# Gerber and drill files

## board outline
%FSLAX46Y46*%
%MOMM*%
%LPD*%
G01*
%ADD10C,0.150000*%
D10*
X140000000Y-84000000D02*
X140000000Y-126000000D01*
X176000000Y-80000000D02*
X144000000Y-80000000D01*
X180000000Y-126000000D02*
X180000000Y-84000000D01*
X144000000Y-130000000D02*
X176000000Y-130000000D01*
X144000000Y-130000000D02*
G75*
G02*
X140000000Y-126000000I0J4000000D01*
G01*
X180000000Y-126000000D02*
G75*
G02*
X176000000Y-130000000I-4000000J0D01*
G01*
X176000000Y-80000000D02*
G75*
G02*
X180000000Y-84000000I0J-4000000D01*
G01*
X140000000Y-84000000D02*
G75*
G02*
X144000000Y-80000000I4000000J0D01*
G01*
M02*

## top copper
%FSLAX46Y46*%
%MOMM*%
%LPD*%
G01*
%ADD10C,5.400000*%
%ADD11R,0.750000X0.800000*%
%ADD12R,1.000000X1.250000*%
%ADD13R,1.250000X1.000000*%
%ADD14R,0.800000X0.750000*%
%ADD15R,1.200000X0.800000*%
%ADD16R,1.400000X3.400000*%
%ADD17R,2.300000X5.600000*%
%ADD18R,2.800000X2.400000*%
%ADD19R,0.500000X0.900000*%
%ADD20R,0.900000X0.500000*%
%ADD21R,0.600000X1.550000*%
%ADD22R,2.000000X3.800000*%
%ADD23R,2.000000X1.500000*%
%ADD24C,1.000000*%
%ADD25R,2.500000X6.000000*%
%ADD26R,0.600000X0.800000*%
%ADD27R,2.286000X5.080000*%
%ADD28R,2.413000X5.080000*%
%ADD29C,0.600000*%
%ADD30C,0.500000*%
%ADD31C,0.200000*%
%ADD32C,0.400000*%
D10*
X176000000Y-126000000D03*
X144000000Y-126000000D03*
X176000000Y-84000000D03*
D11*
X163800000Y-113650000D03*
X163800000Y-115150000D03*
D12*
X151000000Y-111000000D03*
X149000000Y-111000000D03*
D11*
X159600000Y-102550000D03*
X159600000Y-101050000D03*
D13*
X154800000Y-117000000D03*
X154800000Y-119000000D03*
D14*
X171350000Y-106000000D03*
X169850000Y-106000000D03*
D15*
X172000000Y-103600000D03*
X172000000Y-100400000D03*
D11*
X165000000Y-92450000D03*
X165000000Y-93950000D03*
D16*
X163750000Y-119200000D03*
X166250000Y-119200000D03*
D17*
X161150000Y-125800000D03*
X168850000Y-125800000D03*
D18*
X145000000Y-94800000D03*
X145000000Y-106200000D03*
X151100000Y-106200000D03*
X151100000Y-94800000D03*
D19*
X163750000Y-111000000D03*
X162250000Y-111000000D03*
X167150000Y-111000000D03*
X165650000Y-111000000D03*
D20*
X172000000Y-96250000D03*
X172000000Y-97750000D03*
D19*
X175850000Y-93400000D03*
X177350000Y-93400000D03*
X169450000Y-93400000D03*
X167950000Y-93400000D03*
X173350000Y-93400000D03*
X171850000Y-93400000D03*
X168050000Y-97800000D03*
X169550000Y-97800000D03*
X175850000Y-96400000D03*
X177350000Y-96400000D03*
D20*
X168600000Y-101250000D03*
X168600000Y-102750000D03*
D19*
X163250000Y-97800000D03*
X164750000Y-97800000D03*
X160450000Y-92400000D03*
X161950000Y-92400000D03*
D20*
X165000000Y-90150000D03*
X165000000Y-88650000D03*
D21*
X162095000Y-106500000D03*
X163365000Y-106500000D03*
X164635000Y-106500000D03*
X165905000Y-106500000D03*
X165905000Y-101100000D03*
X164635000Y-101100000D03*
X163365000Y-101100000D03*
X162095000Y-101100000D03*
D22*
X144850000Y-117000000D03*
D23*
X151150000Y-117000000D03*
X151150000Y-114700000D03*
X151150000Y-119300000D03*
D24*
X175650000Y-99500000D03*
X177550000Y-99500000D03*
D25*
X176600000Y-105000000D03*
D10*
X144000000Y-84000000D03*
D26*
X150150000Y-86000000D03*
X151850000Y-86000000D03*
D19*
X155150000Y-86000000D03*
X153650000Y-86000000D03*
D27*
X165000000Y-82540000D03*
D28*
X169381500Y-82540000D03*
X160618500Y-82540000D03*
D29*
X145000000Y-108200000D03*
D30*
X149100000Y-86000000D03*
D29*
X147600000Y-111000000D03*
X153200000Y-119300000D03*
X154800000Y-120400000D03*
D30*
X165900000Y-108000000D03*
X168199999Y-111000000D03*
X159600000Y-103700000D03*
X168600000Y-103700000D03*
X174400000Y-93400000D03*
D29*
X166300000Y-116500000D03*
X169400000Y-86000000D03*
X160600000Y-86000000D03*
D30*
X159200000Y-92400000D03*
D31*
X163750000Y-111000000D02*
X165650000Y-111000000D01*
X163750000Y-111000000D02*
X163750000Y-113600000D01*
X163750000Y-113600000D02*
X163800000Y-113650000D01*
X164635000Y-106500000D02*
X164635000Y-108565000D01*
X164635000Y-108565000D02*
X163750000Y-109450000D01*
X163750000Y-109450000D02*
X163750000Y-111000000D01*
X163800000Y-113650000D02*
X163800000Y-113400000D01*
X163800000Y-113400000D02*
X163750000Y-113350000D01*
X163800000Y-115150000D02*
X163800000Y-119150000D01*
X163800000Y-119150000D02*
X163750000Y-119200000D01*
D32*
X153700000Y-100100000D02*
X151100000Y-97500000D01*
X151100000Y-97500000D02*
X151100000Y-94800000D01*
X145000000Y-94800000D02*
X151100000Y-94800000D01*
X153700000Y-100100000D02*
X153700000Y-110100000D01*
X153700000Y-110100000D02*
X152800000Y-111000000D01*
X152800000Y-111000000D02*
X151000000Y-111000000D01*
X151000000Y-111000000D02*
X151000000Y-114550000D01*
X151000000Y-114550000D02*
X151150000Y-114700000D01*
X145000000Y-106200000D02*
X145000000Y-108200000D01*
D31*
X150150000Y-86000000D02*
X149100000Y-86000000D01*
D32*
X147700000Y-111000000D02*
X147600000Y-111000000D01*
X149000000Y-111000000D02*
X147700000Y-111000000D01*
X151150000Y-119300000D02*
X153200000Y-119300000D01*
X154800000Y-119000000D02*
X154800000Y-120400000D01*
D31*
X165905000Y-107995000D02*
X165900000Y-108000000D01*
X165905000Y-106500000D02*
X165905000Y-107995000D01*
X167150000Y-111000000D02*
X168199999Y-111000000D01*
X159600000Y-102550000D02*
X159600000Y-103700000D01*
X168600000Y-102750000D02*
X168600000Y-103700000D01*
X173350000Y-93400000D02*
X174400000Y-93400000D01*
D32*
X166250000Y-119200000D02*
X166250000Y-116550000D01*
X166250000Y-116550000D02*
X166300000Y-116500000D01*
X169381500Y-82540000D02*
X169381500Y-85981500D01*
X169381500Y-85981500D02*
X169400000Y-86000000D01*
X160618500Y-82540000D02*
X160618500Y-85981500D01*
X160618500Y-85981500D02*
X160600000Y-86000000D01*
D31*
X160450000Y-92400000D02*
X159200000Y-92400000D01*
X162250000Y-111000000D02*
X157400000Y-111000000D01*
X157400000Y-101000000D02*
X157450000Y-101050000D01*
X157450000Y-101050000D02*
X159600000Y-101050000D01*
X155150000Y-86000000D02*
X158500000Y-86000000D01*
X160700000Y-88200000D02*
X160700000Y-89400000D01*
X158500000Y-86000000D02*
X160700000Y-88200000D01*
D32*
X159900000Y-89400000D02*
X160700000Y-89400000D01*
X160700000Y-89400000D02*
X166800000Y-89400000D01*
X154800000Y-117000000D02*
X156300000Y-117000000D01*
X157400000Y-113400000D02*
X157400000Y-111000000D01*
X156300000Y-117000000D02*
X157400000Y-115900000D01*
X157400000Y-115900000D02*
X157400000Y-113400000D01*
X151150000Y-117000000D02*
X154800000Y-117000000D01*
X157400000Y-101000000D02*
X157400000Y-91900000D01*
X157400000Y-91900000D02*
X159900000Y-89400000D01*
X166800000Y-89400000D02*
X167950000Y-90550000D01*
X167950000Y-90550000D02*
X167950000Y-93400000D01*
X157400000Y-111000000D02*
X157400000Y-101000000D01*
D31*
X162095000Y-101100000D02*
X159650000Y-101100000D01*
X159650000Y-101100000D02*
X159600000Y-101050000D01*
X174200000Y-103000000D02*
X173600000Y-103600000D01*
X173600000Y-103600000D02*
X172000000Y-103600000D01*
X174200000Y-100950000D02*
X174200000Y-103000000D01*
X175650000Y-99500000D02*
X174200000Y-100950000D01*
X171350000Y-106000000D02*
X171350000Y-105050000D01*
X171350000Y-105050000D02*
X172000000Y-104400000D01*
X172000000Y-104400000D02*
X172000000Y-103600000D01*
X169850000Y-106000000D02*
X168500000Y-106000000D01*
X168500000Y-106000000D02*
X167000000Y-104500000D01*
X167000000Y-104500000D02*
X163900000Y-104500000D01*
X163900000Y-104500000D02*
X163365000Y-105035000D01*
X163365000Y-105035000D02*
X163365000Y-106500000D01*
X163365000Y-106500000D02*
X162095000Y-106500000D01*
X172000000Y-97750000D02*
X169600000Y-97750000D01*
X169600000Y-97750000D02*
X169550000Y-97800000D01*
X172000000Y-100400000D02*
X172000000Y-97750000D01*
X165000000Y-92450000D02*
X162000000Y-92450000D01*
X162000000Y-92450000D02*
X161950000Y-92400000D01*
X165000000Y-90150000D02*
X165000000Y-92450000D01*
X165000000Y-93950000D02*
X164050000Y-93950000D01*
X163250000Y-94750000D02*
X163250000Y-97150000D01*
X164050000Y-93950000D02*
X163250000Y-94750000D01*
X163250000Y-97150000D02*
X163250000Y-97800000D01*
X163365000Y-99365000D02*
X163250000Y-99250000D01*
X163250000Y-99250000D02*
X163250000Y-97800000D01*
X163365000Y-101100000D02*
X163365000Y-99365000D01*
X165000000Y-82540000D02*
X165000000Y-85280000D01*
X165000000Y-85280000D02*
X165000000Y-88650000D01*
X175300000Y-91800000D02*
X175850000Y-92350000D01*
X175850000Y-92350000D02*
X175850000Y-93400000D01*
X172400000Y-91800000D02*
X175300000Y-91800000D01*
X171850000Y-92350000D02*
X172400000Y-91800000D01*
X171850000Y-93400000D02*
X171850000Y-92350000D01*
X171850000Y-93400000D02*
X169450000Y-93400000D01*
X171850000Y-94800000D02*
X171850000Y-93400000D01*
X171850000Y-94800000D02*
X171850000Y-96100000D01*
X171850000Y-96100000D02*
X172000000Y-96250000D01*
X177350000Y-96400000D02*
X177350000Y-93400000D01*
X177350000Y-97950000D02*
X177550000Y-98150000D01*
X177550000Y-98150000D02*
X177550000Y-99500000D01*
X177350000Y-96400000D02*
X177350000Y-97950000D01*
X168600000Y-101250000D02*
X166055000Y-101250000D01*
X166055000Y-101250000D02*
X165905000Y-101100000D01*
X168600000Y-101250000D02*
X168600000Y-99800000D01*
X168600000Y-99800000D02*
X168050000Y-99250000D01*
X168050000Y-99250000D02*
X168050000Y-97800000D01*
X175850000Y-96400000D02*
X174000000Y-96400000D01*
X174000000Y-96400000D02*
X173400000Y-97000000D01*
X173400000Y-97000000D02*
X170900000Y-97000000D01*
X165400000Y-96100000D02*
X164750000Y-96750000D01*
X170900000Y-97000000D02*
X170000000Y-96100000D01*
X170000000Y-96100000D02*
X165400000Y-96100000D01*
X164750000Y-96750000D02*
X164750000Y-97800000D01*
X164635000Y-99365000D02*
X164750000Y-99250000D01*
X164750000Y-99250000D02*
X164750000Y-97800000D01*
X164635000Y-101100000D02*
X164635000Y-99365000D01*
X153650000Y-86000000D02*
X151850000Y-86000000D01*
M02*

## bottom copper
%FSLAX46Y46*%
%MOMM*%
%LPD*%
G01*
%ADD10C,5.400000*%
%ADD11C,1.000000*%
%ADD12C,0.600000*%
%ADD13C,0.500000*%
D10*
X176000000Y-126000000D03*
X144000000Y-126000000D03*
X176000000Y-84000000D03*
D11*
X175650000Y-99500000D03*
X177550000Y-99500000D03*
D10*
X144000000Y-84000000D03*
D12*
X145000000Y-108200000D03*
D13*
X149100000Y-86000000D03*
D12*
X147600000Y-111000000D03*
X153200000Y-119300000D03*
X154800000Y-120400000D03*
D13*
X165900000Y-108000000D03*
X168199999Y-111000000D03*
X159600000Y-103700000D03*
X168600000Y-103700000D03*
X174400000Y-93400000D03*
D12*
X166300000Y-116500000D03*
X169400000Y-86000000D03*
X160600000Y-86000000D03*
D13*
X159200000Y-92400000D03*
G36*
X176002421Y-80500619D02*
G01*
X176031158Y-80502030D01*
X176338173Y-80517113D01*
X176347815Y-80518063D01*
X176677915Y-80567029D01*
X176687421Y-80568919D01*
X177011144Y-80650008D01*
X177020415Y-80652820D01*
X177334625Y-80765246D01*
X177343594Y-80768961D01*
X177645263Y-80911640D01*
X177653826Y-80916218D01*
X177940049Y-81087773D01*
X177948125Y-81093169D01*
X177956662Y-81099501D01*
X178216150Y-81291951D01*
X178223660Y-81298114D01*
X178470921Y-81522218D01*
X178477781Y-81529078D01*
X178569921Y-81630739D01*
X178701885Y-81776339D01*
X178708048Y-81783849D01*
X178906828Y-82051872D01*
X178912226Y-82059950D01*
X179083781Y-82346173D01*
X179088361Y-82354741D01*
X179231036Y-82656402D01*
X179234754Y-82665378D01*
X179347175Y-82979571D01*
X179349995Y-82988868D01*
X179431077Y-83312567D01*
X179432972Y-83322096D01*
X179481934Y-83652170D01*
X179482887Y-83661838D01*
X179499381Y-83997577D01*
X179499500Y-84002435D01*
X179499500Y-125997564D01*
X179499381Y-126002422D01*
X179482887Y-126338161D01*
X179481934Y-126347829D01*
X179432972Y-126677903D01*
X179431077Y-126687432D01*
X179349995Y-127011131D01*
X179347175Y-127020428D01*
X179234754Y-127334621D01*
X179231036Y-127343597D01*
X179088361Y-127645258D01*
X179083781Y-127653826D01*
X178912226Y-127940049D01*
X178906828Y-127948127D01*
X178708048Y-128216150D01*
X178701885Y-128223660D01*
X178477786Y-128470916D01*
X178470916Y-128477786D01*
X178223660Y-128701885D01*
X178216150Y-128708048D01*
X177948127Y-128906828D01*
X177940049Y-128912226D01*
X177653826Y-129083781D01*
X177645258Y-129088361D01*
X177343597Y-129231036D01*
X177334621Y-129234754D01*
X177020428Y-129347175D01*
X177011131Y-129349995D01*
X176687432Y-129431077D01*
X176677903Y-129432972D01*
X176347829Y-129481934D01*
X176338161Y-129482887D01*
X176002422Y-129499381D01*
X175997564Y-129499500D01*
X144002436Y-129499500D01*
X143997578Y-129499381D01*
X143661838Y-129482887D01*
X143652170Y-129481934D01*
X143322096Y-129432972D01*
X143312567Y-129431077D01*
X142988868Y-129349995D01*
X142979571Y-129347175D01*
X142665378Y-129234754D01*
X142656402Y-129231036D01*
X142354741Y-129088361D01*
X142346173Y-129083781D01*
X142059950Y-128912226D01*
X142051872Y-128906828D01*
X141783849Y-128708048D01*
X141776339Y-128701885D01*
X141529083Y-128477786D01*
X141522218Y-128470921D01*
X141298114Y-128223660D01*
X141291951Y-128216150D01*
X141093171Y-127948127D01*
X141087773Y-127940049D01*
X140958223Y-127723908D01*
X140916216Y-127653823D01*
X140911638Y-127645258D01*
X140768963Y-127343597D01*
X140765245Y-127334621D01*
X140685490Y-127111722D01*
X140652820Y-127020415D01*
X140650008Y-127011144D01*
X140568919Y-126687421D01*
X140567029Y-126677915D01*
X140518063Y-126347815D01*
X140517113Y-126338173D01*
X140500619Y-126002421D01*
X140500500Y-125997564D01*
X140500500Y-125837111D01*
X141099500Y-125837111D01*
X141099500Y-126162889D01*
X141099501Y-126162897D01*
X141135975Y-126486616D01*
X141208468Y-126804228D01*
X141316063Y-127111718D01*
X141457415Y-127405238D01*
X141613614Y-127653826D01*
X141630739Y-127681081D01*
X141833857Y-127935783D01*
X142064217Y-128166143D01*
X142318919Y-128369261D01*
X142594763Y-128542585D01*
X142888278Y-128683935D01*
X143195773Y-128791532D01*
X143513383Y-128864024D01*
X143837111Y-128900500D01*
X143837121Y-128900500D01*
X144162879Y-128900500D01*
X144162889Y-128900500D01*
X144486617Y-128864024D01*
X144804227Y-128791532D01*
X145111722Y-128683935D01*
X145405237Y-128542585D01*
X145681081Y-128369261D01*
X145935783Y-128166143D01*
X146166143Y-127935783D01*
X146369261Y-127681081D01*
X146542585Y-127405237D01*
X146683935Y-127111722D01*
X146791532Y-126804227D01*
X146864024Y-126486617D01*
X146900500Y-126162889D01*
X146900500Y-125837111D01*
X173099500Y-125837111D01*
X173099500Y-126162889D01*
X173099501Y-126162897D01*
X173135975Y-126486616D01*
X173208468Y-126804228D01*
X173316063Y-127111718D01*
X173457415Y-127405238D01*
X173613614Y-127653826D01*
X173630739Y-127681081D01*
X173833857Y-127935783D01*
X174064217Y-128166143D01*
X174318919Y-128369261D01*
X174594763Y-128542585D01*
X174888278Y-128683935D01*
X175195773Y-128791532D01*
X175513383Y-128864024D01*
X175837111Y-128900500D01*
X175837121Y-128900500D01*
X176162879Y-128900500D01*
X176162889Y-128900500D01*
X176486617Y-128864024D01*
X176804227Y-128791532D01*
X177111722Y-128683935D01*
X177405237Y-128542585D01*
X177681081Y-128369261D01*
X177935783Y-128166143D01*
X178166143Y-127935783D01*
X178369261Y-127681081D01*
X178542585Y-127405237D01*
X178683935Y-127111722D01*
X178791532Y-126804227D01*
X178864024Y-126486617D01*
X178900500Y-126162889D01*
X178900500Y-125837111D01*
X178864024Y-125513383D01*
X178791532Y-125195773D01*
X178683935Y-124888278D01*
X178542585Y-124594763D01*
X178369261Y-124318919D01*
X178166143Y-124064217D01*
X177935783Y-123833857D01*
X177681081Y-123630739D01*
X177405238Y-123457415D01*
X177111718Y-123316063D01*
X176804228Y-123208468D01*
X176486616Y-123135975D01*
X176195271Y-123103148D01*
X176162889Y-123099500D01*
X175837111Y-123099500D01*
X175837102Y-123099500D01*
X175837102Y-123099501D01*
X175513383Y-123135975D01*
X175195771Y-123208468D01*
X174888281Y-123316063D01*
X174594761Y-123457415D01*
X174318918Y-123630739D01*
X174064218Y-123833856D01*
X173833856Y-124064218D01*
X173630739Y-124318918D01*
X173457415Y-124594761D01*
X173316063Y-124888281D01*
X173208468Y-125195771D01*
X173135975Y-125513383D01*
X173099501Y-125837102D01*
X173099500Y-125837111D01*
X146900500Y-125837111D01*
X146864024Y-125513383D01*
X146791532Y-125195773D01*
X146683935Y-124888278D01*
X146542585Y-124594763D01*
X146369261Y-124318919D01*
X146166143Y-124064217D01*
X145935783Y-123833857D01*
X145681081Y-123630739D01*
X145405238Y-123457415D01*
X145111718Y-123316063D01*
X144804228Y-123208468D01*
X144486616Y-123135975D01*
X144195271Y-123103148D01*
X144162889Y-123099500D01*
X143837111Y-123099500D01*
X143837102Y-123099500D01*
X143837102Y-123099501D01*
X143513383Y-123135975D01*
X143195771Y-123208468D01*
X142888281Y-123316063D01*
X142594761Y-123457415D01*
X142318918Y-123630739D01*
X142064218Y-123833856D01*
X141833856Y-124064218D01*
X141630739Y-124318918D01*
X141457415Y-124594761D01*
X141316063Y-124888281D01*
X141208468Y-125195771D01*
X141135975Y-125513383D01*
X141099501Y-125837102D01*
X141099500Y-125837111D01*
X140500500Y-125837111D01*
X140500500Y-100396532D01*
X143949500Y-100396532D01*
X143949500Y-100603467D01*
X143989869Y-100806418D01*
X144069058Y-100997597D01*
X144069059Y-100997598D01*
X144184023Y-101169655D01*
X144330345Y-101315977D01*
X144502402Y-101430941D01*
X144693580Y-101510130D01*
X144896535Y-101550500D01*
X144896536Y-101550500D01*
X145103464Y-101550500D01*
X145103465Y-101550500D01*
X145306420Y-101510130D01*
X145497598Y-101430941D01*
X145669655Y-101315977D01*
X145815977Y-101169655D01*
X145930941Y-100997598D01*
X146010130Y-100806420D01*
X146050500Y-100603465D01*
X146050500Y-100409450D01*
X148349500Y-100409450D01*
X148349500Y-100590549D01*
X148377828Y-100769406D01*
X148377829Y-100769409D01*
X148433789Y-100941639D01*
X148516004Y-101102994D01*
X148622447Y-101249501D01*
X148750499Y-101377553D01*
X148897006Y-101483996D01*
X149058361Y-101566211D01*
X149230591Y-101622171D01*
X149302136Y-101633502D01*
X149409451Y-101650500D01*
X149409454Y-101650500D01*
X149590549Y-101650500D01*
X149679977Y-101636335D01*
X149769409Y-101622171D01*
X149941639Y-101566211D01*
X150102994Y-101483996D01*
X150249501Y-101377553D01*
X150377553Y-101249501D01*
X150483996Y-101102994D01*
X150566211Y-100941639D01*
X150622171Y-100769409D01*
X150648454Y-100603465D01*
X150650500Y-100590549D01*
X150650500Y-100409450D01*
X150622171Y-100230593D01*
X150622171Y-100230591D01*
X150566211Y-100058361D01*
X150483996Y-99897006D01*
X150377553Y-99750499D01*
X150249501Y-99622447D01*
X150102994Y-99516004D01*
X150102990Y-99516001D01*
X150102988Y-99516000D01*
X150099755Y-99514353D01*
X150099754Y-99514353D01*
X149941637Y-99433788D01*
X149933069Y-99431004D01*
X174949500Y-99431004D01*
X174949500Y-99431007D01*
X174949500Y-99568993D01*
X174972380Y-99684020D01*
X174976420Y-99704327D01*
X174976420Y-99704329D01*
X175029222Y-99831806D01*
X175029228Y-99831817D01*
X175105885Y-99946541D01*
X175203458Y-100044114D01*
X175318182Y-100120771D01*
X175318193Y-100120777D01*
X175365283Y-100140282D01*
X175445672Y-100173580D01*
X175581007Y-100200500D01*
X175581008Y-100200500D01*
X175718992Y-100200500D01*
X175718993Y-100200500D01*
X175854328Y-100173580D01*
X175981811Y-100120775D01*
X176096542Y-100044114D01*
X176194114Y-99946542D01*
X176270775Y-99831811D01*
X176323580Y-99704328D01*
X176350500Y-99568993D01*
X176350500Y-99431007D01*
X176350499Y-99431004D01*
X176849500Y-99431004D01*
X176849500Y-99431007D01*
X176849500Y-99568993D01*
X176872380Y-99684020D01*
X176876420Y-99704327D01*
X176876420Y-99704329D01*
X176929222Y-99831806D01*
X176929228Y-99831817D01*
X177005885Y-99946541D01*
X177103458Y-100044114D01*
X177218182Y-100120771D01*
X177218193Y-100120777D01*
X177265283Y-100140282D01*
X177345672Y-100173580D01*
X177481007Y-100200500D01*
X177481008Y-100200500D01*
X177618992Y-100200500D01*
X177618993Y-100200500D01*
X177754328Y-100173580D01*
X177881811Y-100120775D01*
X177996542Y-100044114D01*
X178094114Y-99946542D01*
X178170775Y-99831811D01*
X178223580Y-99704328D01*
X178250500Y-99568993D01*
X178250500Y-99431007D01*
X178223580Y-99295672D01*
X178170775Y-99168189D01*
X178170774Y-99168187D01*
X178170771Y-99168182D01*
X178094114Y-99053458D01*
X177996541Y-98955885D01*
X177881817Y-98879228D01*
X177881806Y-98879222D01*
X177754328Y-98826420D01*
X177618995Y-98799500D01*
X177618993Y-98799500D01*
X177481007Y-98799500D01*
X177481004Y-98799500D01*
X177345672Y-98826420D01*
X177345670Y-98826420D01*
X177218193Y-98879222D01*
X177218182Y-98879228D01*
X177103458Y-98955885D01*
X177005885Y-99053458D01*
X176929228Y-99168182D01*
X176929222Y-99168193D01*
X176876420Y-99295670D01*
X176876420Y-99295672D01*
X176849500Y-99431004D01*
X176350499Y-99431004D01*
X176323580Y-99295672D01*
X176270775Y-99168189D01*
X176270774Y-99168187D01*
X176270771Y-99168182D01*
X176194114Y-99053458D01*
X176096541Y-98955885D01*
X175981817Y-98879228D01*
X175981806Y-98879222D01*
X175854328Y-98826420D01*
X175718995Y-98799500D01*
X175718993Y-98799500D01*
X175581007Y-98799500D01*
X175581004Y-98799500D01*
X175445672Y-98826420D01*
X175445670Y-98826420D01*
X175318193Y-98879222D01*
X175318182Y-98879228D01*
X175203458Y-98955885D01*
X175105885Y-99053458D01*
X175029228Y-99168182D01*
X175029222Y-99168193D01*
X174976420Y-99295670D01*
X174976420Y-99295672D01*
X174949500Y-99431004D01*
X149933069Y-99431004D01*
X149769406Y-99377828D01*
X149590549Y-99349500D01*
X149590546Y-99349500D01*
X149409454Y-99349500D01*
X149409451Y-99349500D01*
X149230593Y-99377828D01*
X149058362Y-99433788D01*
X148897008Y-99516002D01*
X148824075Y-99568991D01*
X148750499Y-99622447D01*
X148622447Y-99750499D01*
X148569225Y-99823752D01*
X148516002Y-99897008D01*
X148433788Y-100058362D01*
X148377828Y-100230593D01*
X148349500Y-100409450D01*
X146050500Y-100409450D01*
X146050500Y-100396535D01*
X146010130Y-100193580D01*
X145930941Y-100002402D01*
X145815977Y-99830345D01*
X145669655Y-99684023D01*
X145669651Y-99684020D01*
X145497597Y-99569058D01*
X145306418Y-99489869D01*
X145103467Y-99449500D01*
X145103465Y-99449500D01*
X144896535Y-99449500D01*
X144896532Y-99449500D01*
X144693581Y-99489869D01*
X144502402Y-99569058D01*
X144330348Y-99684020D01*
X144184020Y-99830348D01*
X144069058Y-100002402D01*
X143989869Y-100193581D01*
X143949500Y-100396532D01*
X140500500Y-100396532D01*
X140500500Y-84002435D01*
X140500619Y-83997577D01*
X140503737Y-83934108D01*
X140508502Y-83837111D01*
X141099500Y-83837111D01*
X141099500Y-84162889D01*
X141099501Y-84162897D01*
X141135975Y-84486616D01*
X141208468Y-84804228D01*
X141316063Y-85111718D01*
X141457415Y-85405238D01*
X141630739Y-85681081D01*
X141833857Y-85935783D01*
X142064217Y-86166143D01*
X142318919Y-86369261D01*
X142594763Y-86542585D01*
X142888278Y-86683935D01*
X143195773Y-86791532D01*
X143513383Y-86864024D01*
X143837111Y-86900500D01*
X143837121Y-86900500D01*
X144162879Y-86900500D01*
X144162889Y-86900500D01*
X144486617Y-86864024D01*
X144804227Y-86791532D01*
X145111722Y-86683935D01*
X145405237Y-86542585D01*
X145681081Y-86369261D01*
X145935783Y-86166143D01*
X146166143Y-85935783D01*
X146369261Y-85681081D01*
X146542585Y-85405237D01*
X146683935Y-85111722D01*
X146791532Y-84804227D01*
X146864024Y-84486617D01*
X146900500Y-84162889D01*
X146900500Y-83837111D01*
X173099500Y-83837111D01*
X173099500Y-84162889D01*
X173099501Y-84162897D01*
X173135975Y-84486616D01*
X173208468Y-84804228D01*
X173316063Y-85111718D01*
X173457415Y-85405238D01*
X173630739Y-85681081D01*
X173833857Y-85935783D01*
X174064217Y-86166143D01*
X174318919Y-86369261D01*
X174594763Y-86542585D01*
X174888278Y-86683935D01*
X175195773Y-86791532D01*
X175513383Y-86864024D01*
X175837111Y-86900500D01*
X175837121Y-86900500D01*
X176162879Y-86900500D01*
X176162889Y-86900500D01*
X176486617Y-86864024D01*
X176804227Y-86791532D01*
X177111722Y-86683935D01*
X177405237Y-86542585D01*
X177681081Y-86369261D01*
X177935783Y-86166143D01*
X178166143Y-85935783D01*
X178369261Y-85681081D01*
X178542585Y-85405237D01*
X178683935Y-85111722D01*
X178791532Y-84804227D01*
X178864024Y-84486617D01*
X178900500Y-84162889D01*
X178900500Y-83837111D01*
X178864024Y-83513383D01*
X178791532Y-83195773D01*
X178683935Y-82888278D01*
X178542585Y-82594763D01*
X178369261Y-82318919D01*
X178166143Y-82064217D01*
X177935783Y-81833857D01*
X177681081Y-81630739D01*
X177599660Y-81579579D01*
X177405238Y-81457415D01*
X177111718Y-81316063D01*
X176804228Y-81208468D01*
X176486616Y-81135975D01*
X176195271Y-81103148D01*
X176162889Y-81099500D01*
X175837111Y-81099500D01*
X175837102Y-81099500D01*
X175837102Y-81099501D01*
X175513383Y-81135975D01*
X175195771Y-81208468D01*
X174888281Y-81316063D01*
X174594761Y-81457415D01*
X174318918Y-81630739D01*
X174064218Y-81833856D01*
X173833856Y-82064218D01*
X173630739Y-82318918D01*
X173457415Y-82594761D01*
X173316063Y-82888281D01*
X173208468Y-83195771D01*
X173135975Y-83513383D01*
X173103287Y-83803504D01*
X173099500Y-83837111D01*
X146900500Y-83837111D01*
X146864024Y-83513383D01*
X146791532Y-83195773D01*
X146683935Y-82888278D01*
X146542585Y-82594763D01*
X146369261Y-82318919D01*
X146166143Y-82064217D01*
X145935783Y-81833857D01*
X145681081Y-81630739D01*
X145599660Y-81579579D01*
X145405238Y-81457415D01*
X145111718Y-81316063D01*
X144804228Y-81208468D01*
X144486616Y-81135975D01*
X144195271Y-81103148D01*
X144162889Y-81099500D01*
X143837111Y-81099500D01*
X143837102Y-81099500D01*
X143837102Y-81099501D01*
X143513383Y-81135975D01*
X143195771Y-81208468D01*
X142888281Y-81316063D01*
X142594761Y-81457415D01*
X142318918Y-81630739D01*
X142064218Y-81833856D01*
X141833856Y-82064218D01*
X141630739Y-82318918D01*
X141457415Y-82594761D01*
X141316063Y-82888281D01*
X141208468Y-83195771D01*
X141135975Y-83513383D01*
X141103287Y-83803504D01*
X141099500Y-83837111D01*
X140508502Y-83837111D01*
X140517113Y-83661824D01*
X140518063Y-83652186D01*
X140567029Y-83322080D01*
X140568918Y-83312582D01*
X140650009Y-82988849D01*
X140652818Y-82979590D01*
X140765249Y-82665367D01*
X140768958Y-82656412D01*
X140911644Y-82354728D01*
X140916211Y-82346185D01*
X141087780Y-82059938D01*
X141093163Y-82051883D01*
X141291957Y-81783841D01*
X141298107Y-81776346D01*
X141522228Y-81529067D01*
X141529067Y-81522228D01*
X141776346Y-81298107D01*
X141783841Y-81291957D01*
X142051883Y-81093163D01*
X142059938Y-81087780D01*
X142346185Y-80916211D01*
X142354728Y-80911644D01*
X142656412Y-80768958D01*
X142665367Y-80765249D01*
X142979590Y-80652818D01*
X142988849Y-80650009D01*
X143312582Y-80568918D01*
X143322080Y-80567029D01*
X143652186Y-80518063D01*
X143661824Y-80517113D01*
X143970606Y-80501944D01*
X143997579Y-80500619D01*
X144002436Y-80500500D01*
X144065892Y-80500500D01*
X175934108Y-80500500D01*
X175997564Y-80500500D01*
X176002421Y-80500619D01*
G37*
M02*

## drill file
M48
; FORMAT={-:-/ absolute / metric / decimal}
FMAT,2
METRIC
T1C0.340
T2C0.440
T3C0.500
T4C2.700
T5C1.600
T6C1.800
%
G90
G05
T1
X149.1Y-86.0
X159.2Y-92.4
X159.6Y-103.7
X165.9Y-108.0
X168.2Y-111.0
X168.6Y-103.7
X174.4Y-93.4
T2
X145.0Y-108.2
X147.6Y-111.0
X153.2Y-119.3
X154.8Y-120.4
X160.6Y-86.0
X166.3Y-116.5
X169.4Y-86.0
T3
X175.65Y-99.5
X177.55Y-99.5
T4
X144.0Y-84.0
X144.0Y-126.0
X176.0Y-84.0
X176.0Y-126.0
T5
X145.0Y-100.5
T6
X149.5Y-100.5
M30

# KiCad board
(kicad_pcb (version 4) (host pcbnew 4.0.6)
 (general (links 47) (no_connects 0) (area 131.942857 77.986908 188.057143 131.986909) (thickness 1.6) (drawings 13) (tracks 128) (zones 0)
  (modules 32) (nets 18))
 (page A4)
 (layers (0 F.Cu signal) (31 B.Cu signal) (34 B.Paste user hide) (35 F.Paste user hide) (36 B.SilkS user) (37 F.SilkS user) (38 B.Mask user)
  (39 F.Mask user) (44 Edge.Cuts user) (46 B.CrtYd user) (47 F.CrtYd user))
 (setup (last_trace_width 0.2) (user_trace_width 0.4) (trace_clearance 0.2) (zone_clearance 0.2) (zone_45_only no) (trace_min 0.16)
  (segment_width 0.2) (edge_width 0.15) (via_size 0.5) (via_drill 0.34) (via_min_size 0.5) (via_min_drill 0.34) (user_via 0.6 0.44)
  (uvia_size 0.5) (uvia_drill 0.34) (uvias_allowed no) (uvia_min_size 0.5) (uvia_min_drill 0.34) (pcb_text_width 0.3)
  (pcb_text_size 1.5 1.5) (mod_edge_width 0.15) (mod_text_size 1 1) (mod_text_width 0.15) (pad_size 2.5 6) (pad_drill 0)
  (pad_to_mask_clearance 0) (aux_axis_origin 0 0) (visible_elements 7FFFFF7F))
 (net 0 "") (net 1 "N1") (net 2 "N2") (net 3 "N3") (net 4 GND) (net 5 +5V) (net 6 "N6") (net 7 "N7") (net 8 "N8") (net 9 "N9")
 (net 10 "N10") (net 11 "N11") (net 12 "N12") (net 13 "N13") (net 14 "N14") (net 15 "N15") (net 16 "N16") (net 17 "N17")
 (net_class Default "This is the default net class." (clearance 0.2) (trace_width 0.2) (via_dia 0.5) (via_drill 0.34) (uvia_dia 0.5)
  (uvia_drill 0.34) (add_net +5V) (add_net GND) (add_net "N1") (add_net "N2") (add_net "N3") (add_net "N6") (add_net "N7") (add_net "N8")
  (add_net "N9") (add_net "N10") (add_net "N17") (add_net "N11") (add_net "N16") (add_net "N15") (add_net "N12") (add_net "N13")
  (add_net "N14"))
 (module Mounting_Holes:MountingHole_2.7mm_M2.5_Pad (layer F.Cu) (at 176 126)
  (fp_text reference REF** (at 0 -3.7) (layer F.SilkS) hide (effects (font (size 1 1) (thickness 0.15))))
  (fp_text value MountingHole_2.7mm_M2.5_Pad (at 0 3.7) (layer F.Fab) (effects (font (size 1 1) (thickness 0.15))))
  (pad 1 thru_hole circle (at 0 0) (size 5.4 5.4) (drill 2.7) (layers *.Cu *.Mask)))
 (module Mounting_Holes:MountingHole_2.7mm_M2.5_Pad (layer F.Cu) (at 144 126)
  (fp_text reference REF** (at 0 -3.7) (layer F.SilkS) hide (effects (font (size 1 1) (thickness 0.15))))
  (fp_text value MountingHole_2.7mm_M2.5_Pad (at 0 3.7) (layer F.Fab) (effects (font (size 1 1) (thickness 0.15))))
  (pad 1 thru_hole circle (at 0 0) (size 5.4 5.4) (drill 2.7) (layers *.Cu *.Mask)))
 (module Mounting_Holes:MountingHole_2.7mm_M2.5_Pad (layer F.Cu) (at 176 84)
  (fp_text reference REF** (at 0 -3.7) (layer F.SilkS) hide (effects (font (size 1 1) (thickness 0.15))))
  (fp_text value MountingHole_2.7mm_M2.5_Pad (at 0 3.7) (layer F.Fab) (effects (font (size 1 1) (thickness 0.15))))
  (pad 1 thru_hole circle (at 0 0) (size 5.4 5.4) (drill 2.7) (layers *.Cu *.Mask)))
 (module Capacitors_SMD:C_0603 (layer F.Cu) (at 163.8 114.4 270)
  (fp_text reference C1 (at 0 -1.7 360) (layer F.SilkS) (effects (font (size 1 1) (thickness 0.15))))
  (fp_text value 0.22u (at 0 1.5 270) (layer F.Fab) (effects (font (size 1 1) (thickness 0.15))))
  (pad 1 smd rect (at -0.75 0 270) (size 0.8 0.75) (layers F.Cu F.Paste F.Mask) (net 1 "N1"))
  (pad 2 smd rect (at 0.75 0 270) (size 0.8 0.75) (layers F.Cu F.Paste F.Mask) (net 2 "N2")))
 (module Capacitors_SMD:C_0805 (layer F.Cu) (at 150 111 180)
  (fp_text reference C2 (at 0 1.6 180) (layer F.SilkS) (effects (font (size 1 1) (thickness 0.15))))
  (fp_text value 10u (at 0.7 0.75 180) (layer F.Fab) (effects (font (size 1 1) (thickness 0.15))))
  (pad 1 smd rect (at -1 0 180) (size 1 1.25) (layers F.Cu F.Paste F.Mask) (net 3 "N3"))
  (pad 2 smd rect (at 1 0 180) (size 1 1.25) (layers F.Cu F.Paste F.Mask) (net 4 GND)))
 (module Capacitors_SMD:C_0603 (layer F.Cu) (at 159.6 101.8 90)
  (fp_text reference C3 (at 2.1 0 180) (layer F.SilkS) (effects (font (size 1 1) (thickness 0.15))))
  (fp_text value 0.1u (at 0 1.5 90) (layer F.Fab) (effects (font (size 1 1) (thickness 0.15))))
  (pad 1 smd rect (at -0.75 0 90) (size 0.8 0.75) (layers F.Cu F.Paste F.Mask) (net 4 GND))
  (pad 2 smd rect (at 0.75 0 90) (size 0.8 0.75) (layers F.Cu F.Paste F.Mask) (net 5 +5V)))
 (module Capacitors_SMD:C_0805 (layer F.Cu) (at 154.8 118 270)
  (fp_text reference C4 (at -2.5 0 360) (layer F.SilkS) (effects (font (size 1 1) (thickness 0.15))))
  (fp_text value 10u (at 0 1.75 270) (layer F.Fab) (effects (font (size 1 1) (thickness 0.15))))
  (pad 1 smd rect (at -1 0 270) (size 1 1.25) (layers F.Cu F.Paste F.Mask) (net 5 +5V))
  (pad 2 smd rect (at 1 0 270) (size 1 1.25) (layers F.Cu F.Paste F.Mask) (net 4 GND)))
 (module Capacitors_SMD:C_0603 (layer F.Cu) (at 170.6 106 180)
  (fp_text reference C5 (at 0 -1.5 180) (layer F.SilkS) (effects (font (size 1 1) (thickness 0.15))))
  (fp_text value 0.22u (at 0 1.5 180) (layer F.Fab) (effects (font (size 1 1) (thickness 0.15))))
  (pad 1 smd rect (at -0.75 0 180) (size 0.8 0.75) (layers F.Cu F.Paste F.Mask) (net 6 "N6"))
  (pad 2 smd rect (at 0.75 0 180) (size 0.8 0.75) (layers F.Cu F.Paste F.Mask) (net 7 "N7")))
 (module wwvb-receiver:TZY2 (layer F.Cu) (at 172 102 270)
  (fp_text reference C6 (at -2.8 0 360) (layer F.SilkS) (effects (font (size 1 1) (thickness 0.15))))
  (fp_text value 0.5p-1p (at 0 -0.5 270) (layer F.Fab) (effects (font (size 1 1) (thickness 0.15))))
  (pad 2 smd rect (at 1.6 0 270) (size 0.8 1.2) (layers F.Cu F.Paste F.Mask) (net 6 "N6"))
  (pad 1 smd rect (at -1.6 0 270) (size 0.8 1.2) (layers F.Cu F.Paste F.Mask) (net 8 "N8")))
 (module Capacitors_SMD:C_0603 (layer F.Cu) (at 165 93.2 270)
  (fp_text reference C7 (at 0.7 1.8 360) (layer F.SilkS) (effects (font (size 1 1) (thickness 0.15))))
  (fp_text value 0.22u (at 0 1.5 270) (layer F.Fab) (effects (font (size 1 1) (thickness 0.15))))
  (pad 1 smd rect (at -0.75 0 270) (size 0.8 0.75) (layers F.Cu F.Paste F.Mask) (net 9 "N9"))
  (pad 2 smd rect (at 0.75 0 270) (size 0.8 0.75) (layers F.Cu F.Paste F.Mask) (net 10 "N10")))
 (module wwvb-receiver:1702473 (layer F.Cu) (at 165 119.2)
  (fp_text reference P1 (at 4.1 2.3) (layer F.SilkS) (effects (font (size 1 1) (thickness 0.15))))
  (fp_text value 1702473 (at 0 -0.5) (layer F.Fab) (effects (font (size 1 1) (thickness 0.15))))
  (pad 1 smd rect (at -1.25 0) (size 1.4 3.4) (layers F.Cu F.Paste F.Mask) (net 2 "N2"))
  (pad 2 smd rect (at 1.25 0) (size 1.4 3.4) (layers F.Cu F.Paste F.Mask) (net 4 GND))
  (pad "" smd rect (at -3.85 6.6) (size 2.3 5.6) (layers F.Cu F.Paste F.Mask))
  (pad "" smd rect (at 3.85 6.6) (size 2.3 5.6) (layers F.Cu F.Paste F.Mask)))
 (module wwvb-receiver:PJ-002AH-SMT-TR (layer F.Cu) (at 140 100.5)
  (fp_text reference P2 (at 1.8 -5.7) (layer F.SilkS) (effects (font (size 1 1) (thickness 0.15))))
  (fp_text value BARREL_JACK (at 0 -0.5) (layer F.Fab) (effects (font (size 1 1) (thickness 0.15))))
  (pad 1 smd rect (at 5 -5.7) (size 2.8 2.4) (layers F.Cu F.Paste F.Mask) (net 3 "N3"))
  (pad 2 smd rect (at 5 5.7) (size 2.8 2.4) (layers F.Cu F.Paste F.Mask) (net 4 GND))
  (pad 3 smd rect (at 11.1 5.7) (size 2.8 2.4) (layers F.Cu F.Paste F.Mask) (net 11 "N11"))
  (pad 1 smd rect (at 11.1 -5.7) (size 2.8 2.4) (layers F.Cu F.Paste F.Mask) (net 3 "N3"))
  (pad "" np_thru_hole circle (at 5 0) (size 1.6 1.6) (drill 1.6) (layers *.Cu *.Mask))
  (pad "" np_thru_hole circle (at 9.5 0) (size 1.8 1.8) (drill 1.8) (layers *.Cu *.Mask)))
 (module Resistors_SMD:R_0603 (layer F.Cu) (at 163 111 180)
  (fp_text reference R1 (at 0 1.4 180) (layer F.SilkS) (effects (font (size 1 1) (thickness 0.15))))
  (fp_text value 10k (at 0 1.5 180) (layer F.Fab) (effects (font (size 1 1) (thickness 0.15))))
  (pad 1 smd rect (at -0.75 0 180) (size 0.5 0.9) (layers F.Cu F.Paste F.Mask) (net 1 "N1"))
  (pad 2 smd rect (at 0.75 0 180) (size 0.5 0.9) (layers F.Cu F.Paste F.Mask) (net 5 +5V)))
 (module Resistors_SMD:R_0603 (layer F.Cu) (at 166.4 111 180)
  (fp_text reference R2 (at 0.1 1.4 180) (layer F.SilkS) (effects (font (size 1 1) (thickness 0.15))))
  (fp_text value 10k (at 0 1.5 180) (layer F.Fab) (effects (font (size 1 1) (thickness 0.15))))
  (pad 1 smd rect (at -0.75 0 180) (size 0.5 0.9) (layers F.Cu F.Paste F.Mask) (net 4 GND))
  (pad 2 smd rect (at 0.75 0 180) (size 0.5 0.9) (layers F.Cu F.Paste F.Mask) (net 1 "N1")))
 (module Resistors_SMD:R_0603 (layer F.Cu) (at 172 97 270)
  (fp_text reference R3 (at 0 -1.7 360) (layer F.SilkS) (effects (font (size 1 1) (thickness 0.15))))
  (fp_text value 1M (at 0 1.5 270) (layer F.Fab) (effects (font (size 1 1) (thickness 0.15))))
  (pad 1 smd rect (at -0.75 0 270) (size 0.5 0.9) (layers F.Cu F.Paste F.Mask) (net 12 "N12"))
  (pad 2 smd rect (at 0.75 0 270) (size 0.5 0.9) (layers F.Cu F.Paste F.Mask) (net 8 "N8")))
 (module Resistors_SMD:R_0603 (layer F.Cu) (at 176.6 93.4)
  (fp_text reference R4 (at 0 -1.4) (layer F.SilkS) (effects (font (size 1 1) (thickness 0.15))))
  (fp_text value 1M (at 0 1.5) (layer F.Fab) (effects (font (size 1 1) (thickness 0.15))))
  (pad 1 smd rect (at -0.75 0) (size 0.5 0.9) (layers F.Cu F.Paste F.Mask) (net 12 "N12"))
  (pad 2 smd rect (at 0.75 0) (size 0.5 0.9) (layers F.Cu F.Paste F.Mask) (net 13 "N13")))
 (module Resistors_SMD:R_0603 (layer F.Cu) (at 168.7 93.4 180)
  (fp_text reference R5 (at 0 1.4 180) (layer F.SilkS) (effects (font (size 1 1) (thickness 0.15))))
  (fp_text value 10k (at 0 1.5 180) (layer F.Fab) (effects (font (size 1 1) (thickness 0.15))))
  (pad 1 smd rect (at -0.75 0 180) (size 0.5 0.9) (layers F.Cu F.Paste F.Mask) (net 12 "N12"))
  (pad 2 smd rect (at 0.75 0 180) (size 0.5 0.9) (layers F.Cu F.Paste F.Mask) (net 5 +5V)))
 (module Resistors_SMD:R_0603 (layer F.Cu) (at 172.6 93.4 180)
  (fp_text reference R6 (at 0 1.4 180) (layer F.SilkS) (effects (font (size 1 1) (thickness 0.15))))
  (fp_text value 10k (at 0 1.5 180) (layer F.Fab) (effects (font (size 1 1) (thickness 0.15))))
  (pad 1 smd rect (at -0.75 0 180) (size 0.5 0.9) (layers F.Cu F.Paste F.Mask) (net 4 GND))
  (pad 2 smd rect (at 0.75 0 180) (size 0.5 0.9) (layers F.Cu F.Paste F.Mask) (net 12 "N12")))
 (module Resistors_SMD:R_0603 (layer F.Cu) (at 168.8 97.8)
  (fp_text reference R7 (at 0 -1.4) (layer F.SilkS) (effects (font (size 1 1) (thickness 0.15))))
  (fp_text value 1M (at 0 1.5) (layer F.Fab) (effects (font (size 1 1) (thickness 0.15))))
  (pad 1 smd rect (at -0.75 0) (size 0.5 0.9) (layers F.Cu F.Paste F.Mask) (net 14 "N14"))
  (pad 2 smd rect (at 0.75 0) (size 0.5 0.9) (layers F.Cu F.Paste F.Mask) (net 8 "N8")))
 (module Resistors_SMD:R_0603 (layer F.Cu) (at 176.6 96.4)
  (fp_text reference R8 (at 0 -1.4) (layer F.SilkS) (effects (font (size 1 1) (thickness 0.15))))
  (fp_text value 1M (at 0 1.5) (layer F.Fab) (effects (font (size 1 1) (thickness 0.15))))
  (pad 1 smd rect (at -0.75 0) (size 0.5 0.9) (layers F.Cu F.Paste F.Mask) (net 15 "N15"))
  (pad 2 smd rect (at 0.75 0) (size 0.5 0.9) (layers F.Cu F.Paste F.Mask) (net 13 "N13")))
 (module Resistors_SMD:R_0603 (layer F.Cu) (at 168.6 102 270)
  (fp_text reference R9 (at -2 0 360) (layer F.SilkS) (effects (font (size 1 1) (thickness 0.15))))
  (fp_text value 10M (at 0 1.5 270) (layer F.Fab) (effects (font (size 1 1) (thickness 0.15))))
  (pad 1 smd rect (at -0.75 0 270) (size 0.5 0.9) (layers F.Cu F.Paste F.Mask) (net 14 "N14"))
  (pad 2 smd rect (at 0.75 0 270) (size 0.5 0.9) (layers F.Cu F.Paste F.Mask) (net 4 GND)))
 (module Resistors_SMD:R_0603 (layer F.Cu) (at 164 97.8)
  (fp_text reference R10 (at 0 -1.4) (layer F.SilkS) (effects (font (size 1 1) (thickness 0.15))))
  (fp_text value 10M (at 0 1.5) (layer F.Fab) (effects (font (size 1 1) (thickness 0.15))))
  (pad 1 smd rect (at -0.75 0) (size 0.5 0.9) (layers F.Cu F.Paste F.Mask) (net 10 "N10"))
  (pad 2 smd rect (at 0.75 0) (size 0.5 0.9) (layers F.Cu F.Paste F.Mask) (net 15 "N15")))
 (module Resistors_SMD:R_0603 (layer F.Cu) (at 161.2 92.4)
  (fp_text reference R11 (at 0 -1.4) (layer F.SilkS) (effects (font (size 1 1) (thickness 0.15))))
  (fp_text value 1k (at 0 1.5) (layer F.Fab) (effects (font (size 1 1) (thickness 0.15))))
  (pad 1 smd rect (at -0.75 0) (size 0.5 0.9) (layers F.Cu F.Paste F.Mask) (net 4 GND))
  (pad 2 smd rect (at 0.75 0) (size 0.5 0.9) (layers F.Cu F.Paste F.Mask) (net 9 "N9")))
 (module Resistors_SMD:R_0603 (layer F.Cu) (at 165 89.4 90)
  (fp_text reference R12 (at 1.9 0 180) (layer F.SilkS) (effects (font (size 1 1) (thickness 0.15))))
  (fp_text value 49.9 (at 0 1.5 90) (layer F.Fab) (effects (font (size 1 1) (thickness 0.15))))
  (pad 1 smd rect (at -0.75 0 90) (size 0.5 0.9) (layers F.Cu F.Paste F.Mask) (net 9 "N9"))
  (pad 2 smd rect (at 0.75 0 90) (size 0.5 0.9) (layers F.Cu F.Paste F.Mask) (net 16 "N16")))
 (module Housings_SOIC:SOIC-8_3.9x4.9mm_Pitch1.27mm (layer F.Cu) (at 164 103.8 90)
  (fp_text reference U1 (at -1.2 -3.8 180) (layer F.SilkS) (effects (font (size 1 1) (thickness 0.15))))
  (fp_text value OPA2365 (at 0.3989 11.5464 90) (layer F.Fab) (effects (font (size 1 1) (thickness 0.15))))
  (pad 1 smd rect (at -2.7 -1.905 90) (size 1.55 0.6) (layers F.Cu F.Paste F.Mask) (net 7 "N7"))
  (pad 2 smd rect (at -2.7 -0.635 90) (size 1.55 0.6) (layers F.Cu F.Paste F.Mask) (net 7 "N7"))
  (pad 3 smd rect (at -2.7 0.635 90) (size 1.55 0.6) (layers F.Cu F.Paste F.Mask) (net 1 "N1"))
  (pad 4 smd rect (at -2.7 1.905 90) (size 1.55 0.6) (layers F.Cu F.Paste F.Mask) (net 4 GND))
  (pad 5 smd rect (at 2.7 1.905 90) (size 1.55 0.6) (layers F.Cu F.Paste F.Mask) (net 14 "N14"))
  (pad 6 smd rect (at 2.7 0.635 90) (size 1.55 0.6) (layers F.Cu F.Paste F.Mask) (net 15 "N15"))
  (pad 7 smd rect (at 2.7 -0.635 90) (size 1.55 0.6) (layers F.Cu F.Paste F.Mask) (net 10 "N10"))
  (pad 8 smd rect (at 2.7 -1.905 90) (size 1.55 0.6) (layers F.Cu F.Paste F.Mask) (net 5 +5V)))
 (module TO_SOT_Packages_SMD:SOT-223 (layer F.Cu) (at 148 117 180)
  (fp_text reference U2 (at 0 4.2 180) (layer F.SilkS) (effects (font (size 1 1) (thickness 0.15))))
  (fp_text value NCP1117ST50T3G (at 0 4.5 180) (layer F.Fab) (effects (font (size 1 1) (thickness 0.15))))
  (pad 4 smd rect (at 3.15 0 180) (size 2 3.8) (layers F.Cu F.Paste F.Mask))
  (pad 2 smd rect (at -3.15 0 180) (size 2 1.5) (layers F.Cu F.Paste F.Mask) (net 5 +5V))
  (pad 3 smd rect (at -3.15 2.3 180) (size 2 1.5) (layers F.Cu F.Paste F.Mask) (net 3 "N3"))
  (pad 1 smd rect (at -3.15 -2.3 180) (size 2 1.5) (layers F.Cu F.Paste F.Mask) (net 4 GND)))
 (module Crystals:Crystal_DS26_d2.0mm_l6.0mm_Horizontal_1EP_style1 (layer F.Cu) (at 175.65 99.5)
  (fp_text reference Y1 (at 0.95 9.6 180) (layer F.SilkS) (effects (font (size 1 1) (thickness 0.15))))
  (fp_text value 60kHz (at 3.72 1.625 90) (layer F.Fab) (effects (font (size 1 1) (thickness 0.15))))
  (pad 1 thru_hole circle (at 0 0) (size 1 1) (drill 0.5) (layers *.Cu *.Mask) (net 6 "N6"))
  (pad 2 thru_hole circle (at 1.9 0) (size 1 1) (drill 0.5) (layers *.Cu *.Mask) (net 13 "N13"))
  (pad 3 smd rect (at 0.95 5.5) (size 2.5 6) (layers F.Cu F.Mask)))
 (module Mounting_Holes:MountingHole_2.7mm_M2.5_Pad (layer F.Cu) (at 144 84)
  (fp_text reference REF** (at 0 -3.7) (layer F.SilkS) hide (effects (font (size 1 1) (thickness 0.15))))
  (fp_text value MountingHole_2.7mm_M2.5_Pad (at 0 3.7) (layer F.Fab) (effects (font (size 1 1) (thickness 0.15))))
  (pad 1 thru_hole circle (at 0 0) (size 5.4 5.4) (drill 2.7) (layers *.Cu *.Mask)))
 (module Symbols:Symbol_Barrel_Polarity (layer F.Cu) (at 146.1 91.8)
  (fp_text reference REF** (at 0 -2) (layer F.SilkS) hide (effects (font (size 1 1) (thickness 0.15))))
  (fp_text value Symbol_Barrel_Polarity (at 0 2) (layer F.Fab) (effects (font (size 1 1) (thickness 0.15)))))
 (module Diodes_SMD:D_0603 (layer F.Cu) (at 151 86)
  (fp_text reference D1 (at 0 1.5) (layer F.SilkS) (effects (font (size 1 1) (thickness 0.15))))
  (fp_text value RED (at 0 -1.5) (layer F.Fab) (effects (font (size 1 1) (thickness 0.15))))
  (pad 1 smd rect (at -0.85 0) (size 0.6 0.8) (layers F.Cu F.Paste F.Mask) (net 4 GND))
  (pad 2 smd rect (at 0.85 0) (size 0.6 0.8) (layers F.Cu F.Paste F.Mask) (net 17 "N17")))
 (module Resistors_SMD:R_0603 (layer F.Cu) (at 154.4 86 180)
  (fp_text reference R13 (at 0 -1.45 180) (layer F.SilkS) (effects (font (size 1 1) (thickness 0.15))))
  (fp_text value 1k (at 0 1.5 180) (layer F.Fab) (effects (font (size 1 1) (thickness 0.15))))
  (pad 1 smd rect (at -0.75 0 180) (size 0.5 0.9) (layers F.Cu F.Paste F.Mask) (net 5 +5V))
  (pad 2 smd rect (at 0.75 0 180) (size 0.5 0.9) (layers F.Cu F.Paste F.Mask) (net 17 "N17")))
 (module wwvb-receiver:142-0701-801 (layer F.Cu) (at 165 80)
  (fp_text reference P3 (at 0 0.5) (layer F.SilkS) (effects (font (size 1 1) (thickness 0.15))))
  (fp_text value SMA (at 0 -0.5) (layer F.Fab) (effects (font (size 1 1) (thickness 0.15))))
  (pad 1 smd rect (at 0 2.54) (size 2.286 5.08) (layers F.Cu F.Mask) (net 16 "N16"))
  (pad 2 smd rect (at 4.3815 2.54) (size 2.413 5.08) (layers F.Cu F.Mask) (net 4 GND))
  (pad 2 smd rect (at -4.3815 2.54) (size 2.413 5.08) (layers F.Cu F.Mask) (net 4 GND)))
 (gr_line (start 140 84) (end 140 126) (layer Edge.Cuts) (width 0.15))
 (gr_line (start 176 80) (end 144 80) (layer Edge.Cuts) (width 0.15))
 (gr_line (start 180 126) (end 180 84) (layer Edge.Cuts) (width 0.15))
 (gr_line (start 144 130) (end 176 130) (layer Edge.Cuts) (width 0.15))
 (gr_arc (start 144 126) (end 144 130) (angle 90) (layer Edge.Cuts) (width 0.15))
 (gr_arc (start 176 126) (end 180 126) (angle 90) (layer Edge.Cuts) (width 0.15))
 (gr_arc (start 176 84) (end 176 80) (angle 90) (layer Edge.Cuts) (width 0.15))
 (gr_arc (start 144 84) (end 140 84) (angle 90) (layer Edge.Cuts) (width 0.15))
 (segment (start 163.75 111) (end 165.65 111) (width 0.2) (layer F.Cu) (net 1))
 (segment (start 163.75 111) (end 163.75 113.6) (width 0.2) (layer F.Cu) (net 1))
 (segment (start 163.75 113.6) (end 163.8 113.65) (width 0.2) (layer F.Cu) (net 1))
 (segment (start 164.635 106.5) (end 164.635 108.565) (width 0.2) (layer F.Cu) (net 1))
 (segment (start 164.635 108.565) (end 163.75 109.45) (width 0.2) (layer F.Cu) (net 1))
 (segment (start 163.75 109.45) (end 163.75 111) (width 0.2) (layer F.Cu) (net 1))
 (segment (start 163.8 113.65) (end 163.8 113.4) (width 0.2) (layer F.Cu) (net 1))
 (segment (start 163.8 113.4) (end 163.75 113.35) (width 0.2) (layer F.Cu) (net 1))
 (segment (start 163.8 115.15) (end 163.8 119.15) (width 0.2) (layer F.Cu) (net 2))
 (segment (start 163.8 119.15) (end 163.75 119.2) (width 0.2) (layer F.Cu) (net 2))
 (segment (start 153.7 100.1) (end 151.1 97.5) (width 0.4) (layer F.Cu) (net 3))
 (segment (start 151.1 97.5) (end 151.1 94.8) (width 0.4) (layer F.Cu) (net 3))
 (segment (start 145 94.8) (end 151.1 94.8) (width 0.4) (layer F.Cu) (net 3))
 (segment (start 153.7 100.1) (end 153.7 110.1) (width 0.4) (layer F.Cu) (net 3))
 (segment (start 153.7 110.1) (end 152.8 111) (width 0.4) (layer F.Cu) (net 3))
 (segment (start 152.8 111) (end 151 111) (width 0.4) (layer F.Cu) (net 3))
 (segment (start 151 111) (end 151 114.55) (width 0.4) (layer F.Cu) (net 3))
 (segment (start 151 114.55) (end 151.15 114.7) (width 0.4) (layer F.Cu) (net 3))
 (segment (start 145 106.2) (end 145 108.2) (width 0.4) (layer F.Cu) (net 4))
 (via (at 145 108.2) (size 0.6) (drill 0.44) (layers F.Cu B.Cu) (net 4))
 (segment (start 150.15 86) (end 149.1 86) (width 0.2) (layer F.Cu) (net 4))
 (via (at 149.1 86) (size 0.5) (drill 0.34) (layers F.Cu B.Cu) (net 4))
 (segment (start 147.7 111) (end 147.6 111) (width 0.4) (layer F.Cu) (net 4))
 (via (at 147.6 111) (size 0.6) (drill 0.44) (layers F.Cu B.Cu) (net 4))
 (segment (start 149 111) (end 147.7 111) (width 0.4) (layer F.Cu) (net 4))
 (segment (start 151.15 119.3) (end 153.2 119.3) (width 0.4) (layer F.Cu) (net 4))
 (via (at 153.2 119.3) (size 0.6) (drill 0.44) (layers F.Cu B.Cu) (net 4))
 (segment (start 154.8 119) (end 154.8 120.4) (width 0.4) (layer F.Cu) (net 4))
 (via (at 154.8 120.4) (size 0.6) (drill 0.44) (layers F.Cu B.Cu) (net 4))
 (segment (start 165.905 107.995) (end 165.9 108) (width 0.2) (layer F.Cu) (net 4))
 (segment (start 165.905 106.5) (end 165.905 107.995) (width 0.2) (layer F.Cu) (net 4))
 (via (at 165.9 108) (size 0.5) (drill 0.34) (layers F.Cu B.Cu) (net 4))
 (segment (start 167.15 111) (end 168.199999 111) (width 0.2) (layer F.Cu) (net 4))
 (via (at 168.199999 111) (size 0.5) (drill 0.34) (layers F.Cu B.Cu) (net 4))
 (segment (start 159.6 102.55) (end 159.6 103.7) (width 0.2) (layer F.Cu) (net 4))
 (via (at 159.6 103.7) (size 0.5) (drill 0.34) (layers F.Cu B.Cu) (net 4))
 (segment (start 168.6 102.75) (end 168.6 103.7) (width 0.2) (layer F.Cu) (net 4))
 (via (at 168.6 103.7) (size 0.5) (drill 0.34) (layers F.Cu B.Cu) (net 4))
 (segment (start 173.35 93.4) (end 174.4 93.4) (width 0.2) (layer F.Cu) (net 4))
 (via (at 174.4 93.4) (size 0.5) (drill 0.34) (layers F.Cu B.Cu) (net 4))
 (segment (start 166.25 119.2) (end 166.25 116.55) (width 0.4) (layer F.Cu) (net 4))
 (segment (start 166.25 116.55) (end 166.3 116.5) (width 0.4) (layer F.Cu) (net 4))
 (via (at 166.3 116.5) (size 0.6) (drill 0.44) (layers F.Cu B.Cu) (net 4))
 (segment (start 169.3815 82.54) (end 169.3815 85.9815) (width 0.4) (layer F.Cu) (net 4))
 (segment (start 169.3815 85.9815) (end 169.4 86) (width 0.4) (layer F.Cu) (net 4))
 (via (at 169.4 86) (size 0.6) (drill 0.44) (layers F.Cu B.Cu) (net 4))
 (segment (start 160.6185 82.54) (end 160.6185 85.9815) (width 0.4) (layer F.Cu) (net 4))
 (segment (start 160.6185 85.9815) (end 160.6 86) (width 0.4) (layer F.Cu) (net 4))
 (via (at 160.6 86) (size 0.6) (drill 0.44) (layers F.Cu B.Cu) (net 4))
 (segment (start 160.45 92.4) (end 159.2 92.4) (width 0.2) (layer F.Cu) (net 4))
 (via (at 159.2 92.4) (size 0.5) (drill 0.34) (layers F.Cu B.Cu) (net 4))
 (segment (start 162.25 111) (end 157.4 111) (width 0.2) (layer F.Cu) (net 5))
 (segment (start 157.4 101) (end 157.45 101.05) (width 0.2) (layer F.Cu) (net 5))
 (segment (start 157.45 101.05) (end 159.6 101.05) (width 0.2) (layer F.Cu) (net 5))
 (segment (start 155.15 86) (end 158.5 86) (width 0.2) (layer F.Cu) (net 5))
 (segment (start 160.7 88.2) (end 160.7 89.4) (width 0.2) (layer F.Cu) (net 5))
 (segment (start 158.5 86) (end 160.7 88.2) (width 0.2) (layer F.Cu) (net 5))
 (segment (start 159.9 89.4) (end 160.7 89.4) (width 0.4) (layer F.Cu) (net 5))
 (segment (start 160.7 89.4) (end 166.8 89.4) (width 0.4) (layer F.Cu) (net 5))
 (segment (start 154.8 117) (end 156.3 117) (width 0.4) (layer F.Cu) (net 5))
 (segment (start 157.4 113.4) (end 157.4 111) (width 0.4) (layer F.Cu) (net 5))
 (segment (start 156.3 117) (end 157.4 115.9) (width 0.4) (layer F.Cu) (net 5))
 (segment (start 157.4 115.9) (end 157.4 113.4) (width 0.4) (layer F.Cu) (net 5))
 (segment (start 151.15 117) (end 154.8 117) (width 0.4) (layer F.Cu) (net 5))
 (segment (start 157.4 101) (end 157.4 91.9) (width 0.4) (layer F.Cu) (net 5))
 (segment (start 157.4 91.9) (end 159.9 89.4) (width 0.4) (layer F.Cu) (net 5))
 (segment (start 166.8 89.4) (end 167.95 90.55) (width 0.4) (layer F.Cu) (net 5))
 (segment (start 167.95 90.55) (end 167.95 93.4) (width 0.4) (layer F.Cu) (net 5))
 (segment (start 157.4 111) (end 157.4 101) (width 0.4) (layer F.Cu) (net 5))
 (segment (start 162.095 101.1) (end 159.65 101.1) (width 0.2) (layer F.Cu) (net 5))
 (segment (start 159.65 101.1) (end 159.6 101.05) (width 0.2) (layer F.Cu) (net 5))
 (segment (start 174.2 103) (end 173.6 103.6) (width 0.2) (layer F.Cu) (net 6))
 (segment (start 173.6 103.6) (end 172 103.6) (width 0.2) (layer F.Cu) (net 6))
 (segment (start 174.2 100.95) (end 174.2 103) (width 0.2) (layer F.Cu) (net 6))
 (segment (start 175.65 99.5) (end 174.2 100.95) (width 0.2) (layer F.Cu) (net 6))
 (segment (start 171.35 106) (end 171.35 105.05) (width 0.2) (layer F.Cu) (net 6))
 (segment (start 171.35 105.05) (end 172 104.4) (width 0.2) (layer F.Cu) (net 6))
 (segment (start 172 104.4) (end 172 103.6) (width 0.2) (layer F.Cu) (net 6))
 (segment (start 169.85 106) (end 168.5 106) (width 0.2) (layer F.Cu) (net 7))
 (segment (start 168.5 106) (end 167 104.5) (width 0.2) (layer F.Cu) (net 7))
 (segment (start 167 104.5) (end 163.9 104.5) (width 0.2) (layer F.Cu) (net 7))
 (segment (start 163.9 104.5) (end 163.365 105.035) (width 0.2) (layer F.Cu) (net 7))
 (segment (start 163.365 105.035) (end 163.365 106.5) (width 0.2) (layer F.Cu) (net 7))
 (segment (start 163.365 106.5) (end 162.095 106.5) (width 0.2) (layer F.Cu) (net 7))
 (segment (start 172 97.75) (end 169.6 97.75) (width 0.2) (layer F.Cu) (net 8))
 (segment (start 169.6 97.75) (end 169.55 97.8) (width 0.2) (layer F.Cu) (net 8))
 (segment (start 172 100.4) (end 172 97.75) (width 0.2) (layer F.Cu) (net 8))
 (segment (start 165 92.45) (end 162 92.45) (width 0.2) (layer F.Cu) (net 9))
 (segment (start 162 92.45) (end 161.95 92.4) (width 0.2) (layer F.Cu) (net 9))
 (segment (start 165 90.15) (end 165 92.45) (width 0.2) (layer F.Cu) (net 9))
 (segment (start 165 93.95) (end 164.05 93.95) (width 0.2) (layer F.Cu) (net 10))
 (segment (start 163.25 94.75) (end 163.25 97.15) (width 0.2) (layer F.Cu) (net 10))
 (segment (start 164.05 93.95) (end 163.25 94.75) (width 0.2) (layer F.Cu) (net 10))
 (segment (start 163.25 97.15) (end 163.25 97.8) (width 0.2) (layer F.Cu) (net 10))
 (segment (start 163.365 99.365) (end 163.25 99.25) (width 0.2) (layer F.Cu) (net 10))
 (segment (start 163.25 99.25) (end 163.25 97.8) (width 0.2) (layer F.Cu) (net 10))
 (segment (start 163.365 101.1) (end 163.365 99.365) (width 0.2) (layer F.Cu) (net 10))
 (segment (start 165 82.54) (end 165 85.28) (width 0.2) (layer F.Cu) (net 16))
 (segment (start 165 85.28) (end 165 88.65) (width 0.2) (layer F.Cu) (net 16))
 (segment (start 175.3 91.8) (end 175.85 92.35) (width 0.2) (layer F.Cu) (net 12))
 (segment (start 175.85 92.35) (end 175.85 93.4) (width 0.2) (layer F.Cu) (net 12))
 (segment (start 172.4 91.8) (end 175.3 91.8) (width 0.2) (layer F.Cu) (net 12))
 (segment (start 171.85 92.35) (end 172.4 91.8) (width 0.2) (layer F.Cu) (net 12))
 (segment (start 171.85 93.4) (end 171.85 92.35) (width 0.2) (layer F.Cu) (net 12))
 (segment (start 171.85 93.4) (end 169.45 93.4) (width 0.2) (layer F.Cu) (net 12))
 (segment (start 171.85 94.8) (end 171.85 93.4) (width 0.2) (layer F.Cu) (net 12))
 (segment (start 171.85 94.8) (end 171.85 96.1) (width 0.2) (layer F.Cu) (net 12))
 (segment (start 171.85 96.1) (end 172 96.25) (width 0.2) (layer F.Cu) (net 12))
 (segment (start 177.35 96.4) (end 177.35 93.4) (width 0.2) (layer F.Cu) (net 13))
 (segment (start 177.35 97.95) (end 177.55 98.15) (width 0.2) (layer F.Cu) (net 13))
 (segment (start 177.55 98.15) (end 177.55 99.5) (width 0.2) (layer F.Cu) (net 13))
 (segment (start 177.35 96.4) (end 177.35 97.95) (width 0.2) (layer F.Cu) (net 13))
 (segment (start 168.6 101.25) (end 166.055 101.25) (width 0.2) (layer F.Cu) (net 14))
 (segment (start 166.055 101.25) (end 165.905 101.1) (width 0.2) (layer F.Cu) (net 14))
 (segment (start 168.6 101.25) (end 168.6 99.8) (width 0.2) (layer F.Cu) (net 14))
 (segment (start 168.6 99.8) (end 168.05 99.25) (width 0.2) (layer F.Cu) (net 14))
 (segment (start 168.05 99.25) (end 168.05 97.8) (width 0.2) (layer F.Cu) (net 14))
 (segment (start 175.85 96.4) (end 174 96.4) (width 0.2) (layer F.Cu) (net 15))
 (segment (start 174 96.4) (end 173.4 97) (width 0.2) (layer F.Cu) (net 15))
 (segment (start 173.4 97) (end 170.9 97) (width 0.2) (layer F.Cu) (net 15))
 (segment (start 165.4 96.1) (end 164.75 96.75) (width 0.2) (layer F.Cu) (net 15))
 (segment (start 170.9 97) (end 170 96.1) (width 0.2) (layer F.Cu) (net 15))
 (segment (start 170 96.1) (end 165.4 96.1) (width 0.2) (layer F.Cu) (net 15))
 (segment (start 164.75 96.75) (end 164.75 97.8) (width 0.2) (layer F.Cu) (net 15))
 (segment (start 164.635 99.365) (end 164.75 99.25) (width 0.2) (layer F.Cu) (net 15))
 (segment (start 164.75 99.25) (end 164.75 97.8) (width 0.2) (layer F.Cu) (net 15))
 (segment (start 164.635 101.1) (end 164.635 99.365) (width 0.2) (layer F.Cu) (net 15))
 (segment (start 153.65 86) (end 151.85 86) (width 0.2) (layer F.Cu) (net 17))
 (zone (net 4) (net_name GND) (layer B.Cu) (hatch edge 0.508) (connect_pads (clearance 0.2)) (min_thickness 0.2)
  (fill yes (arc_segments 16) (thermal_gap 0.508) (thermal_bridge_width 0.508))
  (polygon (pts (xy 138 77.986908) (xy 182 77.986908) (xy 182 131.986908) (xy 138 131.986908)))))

